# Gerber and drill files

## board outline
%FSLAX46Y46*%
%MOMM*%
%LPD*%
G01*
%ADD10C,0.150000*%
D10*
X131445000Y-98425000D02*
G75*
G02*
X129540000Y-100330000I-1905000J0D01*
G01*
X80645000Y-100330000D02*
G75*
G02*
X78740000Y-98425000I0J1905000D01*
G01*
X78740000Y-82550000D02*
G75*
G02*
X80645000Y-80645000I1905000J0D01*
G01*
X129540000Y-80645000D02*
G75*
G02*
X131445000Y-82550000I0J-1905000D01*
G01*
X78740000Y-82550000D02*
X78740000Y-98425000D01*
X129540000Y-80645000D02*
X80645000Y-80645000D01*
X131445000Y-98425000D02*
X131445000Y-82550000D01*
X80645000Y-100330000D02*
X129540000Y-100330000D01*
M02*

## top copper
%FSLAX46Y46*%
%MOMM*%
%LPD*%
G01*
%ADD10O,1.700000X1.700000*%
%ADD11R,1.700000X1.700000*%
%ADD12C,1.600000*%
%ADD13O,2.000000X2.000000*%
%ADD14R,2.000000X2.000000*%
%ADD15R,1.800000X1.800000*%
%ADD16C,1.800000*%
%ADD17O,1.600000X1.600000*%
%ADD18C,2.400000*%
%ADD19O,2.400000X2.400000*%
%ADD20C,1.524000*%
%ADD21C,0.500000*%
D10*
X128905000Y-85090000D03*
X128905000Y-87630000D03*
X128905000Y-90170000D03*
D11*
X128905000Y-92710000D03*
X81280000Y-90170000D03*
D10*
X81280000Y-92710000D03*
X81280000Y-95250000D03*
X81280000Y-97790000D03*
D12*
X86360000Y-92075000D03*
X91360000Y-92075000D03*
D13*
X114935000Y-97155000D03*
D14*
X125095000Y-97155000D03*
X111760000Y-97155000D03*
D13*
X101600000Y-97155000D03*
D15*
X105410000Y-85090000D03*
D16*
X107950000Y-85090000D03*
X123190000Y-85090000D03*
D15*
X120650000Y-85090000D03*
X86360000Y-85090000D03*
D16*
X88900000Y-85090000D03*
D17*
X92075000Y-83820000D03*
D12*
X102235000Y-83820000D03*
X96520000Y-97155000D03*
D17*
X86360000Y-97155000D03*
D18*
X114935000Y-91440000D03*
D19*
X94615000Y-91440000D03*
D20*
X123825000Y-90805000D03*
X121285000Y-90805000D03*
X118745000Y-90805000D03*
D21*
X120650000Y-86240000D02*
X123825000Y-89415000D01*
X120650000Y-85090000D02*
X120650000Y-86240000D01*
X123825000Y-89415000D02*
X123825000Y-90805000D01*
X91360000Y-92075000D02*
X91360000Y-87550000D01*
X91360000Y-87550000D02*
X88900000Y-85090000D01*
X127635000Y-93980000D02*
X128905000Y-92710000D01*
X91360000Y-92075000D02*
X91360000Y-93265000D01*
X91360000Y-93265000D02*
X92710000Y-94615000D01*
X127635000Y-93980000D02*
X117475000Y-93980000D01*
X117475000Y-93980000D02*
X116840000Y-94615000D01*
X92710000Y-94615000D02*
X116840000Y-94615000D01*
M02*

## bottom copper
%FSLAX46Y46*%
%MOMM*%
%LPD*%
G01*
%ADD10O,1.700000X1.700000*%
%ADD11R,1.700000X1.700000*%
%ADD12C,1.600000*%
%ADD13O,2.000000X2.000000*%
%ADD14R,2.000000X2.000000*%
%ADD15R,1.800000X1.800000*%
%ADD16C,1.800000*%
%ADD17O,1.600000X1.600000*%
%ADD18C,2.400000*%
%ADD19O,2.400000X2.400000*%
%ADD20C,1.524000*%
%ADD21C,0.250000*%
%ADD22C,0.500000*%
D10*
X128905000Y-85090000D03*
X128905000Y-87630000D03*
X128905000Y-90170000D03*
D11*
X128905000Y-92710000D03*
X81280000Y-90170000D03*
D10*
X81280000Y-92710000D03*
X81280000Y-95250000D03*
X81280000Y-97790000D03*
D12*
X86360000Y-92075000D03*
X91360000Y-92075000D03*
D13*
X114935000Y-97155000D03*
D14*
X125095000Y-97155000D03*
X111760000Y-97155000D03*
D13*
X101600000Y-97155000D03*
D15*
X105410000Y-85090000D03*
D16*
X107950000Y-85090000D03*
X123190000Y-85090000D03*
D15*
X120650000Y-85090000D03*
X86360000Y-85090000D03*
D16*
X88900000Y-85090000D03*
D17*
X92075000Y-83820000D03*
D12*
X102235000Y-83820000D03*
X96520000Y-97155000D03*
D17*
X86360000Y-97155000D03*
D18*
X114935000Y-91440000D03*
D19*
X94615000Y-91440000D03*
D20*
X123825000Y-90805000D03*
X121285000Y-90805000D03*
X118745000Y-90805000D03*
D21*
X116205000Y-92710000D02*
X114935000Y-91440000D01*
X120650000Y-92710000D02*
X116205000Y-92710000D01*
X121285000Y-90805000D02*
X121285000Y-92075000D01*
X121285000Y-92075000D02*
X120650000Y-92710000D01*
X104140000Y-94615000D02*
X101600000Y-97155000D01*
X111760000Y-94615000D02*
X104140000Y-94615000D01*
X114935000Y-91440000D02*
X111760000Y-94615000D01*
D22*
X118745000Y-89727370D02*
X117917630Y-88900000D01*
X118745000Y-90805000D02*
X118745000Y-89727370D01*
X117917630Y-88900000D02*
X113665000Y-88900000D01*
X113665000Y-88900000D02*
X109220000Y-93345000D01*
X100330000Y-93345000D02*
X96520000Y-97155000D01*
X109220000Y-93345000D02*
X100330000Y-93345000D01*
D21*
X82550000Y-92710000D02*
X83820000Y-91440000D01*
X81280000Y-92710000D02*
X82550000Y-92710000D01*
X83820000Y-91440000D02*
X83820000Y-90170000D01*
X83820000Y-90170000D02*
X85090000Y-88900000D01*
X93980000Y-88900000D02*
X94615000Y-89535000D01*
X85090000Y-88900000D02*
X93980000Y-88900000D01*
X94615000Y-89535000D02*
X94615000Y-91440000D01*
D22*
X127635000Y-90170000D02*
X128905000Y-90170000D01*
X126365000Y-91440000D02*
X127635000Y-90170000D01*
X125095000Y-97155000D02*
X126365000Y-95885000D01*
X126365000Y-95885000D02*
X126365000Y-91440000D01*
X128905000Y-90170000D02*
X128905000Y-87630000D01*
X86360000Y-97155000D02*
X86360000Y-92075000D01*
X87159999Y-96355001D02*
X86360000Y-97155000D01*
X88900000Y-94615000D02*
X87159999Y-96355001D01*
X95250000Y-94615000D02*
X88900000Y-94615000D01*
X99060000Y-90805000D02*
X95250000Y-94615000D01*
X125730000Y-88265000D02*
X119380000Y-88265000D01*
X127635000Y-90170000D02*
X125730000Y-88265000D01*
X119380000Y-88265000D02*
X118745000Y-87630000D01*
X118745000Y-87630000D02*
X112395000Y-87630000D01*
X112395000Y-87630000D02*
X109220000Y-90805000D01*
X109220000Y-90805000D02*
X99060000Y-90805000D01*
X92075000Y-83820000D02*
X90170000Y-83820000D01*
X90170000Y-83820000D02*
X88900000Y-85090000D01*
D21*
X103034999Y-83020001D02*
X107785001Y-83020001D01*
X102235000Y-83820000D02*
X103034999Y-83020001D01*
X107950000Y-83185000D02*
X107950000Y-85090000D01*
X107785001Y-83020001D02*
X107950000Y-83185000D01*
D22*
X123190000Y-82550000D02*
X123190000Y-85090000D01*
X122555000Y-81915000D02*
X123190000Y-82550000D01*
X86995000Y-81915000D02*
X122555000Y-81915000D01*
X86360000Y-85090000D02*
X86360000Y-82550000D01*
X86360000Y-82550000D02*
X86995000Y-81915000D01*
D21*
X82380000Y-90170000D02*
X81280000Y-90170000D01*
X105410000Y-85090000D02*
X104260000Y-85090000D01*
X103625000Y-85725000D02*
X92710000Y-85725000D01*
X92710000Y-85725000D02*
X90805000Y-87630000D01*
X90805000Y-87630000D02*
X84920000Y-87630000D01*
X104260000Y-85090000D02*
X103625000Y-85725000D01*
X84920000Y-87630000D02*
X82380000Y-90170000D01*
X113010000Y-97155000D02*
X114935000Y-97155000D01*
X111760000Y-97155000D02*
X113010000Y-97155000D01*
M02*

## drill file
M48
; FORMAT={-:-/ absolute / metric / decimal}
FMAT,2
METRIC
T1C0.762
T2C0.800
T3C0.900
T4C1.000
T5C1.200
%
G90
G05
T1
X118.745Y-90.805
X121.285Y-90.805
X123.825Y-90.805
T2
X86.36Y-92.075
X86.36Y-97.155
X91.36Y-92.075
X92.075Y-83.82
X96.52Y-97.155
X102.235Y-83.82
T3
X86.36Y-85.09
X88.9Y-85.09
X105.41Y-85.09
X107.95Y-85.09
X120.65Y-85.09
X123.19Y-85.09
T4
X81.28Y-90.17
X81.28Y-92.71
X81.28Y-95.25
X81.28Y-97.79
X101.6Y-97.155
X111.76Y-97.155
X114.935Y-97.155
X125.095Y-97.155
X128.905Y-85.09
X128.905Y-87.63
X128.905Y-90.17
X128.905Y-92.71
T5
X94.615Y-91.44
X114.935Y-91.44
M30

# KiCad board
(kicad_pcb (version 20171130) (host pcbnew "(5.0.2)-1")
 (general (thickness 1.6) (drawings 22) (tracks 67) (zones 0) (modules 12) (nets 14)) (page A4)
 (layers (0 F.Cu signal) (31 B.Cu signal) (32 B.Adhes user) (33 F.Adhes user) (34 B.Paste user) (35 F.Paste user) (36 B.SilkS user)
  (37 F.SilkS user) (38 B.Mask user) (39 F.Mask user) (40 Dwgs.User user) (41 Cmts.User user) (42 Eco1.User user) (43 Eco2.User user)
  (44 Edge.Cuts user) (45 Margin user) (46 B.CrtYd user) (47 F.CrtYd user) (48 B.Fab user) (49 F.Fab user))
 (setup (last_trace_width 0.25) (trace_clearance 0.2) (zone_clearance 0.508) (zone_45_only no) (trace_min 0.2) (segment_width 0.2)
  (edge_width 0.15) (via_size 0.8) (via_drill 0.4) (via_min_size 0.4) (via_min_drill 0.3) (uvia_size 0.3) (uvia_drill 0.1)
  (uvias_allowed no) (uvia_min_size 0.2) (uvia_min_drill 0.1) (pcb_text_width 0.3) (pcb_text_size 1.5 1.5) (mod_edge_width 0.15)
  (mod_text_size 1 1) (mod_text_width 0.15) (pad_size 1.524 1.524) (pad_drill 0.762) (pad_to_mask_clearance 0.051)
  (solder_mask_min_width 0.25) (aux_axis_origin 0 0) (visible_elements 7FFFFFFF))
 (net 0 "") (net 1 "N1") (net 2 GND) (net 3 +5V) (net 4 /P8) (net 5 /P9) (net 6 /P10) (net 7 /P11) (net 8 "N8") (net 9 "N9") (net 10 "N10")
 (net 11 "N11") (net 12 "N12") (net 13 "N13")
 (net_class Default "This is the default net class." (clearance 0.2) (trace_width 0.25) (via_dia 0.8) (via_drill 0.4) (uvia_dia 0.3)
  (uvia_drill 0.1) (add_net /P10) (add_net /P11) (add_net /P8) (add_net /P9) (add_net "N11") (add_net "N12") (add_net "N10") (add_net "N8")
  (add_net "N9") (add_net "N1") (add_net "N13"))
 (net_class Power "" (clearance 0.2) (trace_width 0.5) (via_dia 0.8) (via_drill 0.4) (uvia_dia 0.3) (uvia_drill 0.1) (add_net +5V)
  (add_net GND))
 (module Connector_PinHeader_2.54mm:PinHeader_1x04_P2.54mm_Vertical (layer B.Cu) (at 128.905 92.71)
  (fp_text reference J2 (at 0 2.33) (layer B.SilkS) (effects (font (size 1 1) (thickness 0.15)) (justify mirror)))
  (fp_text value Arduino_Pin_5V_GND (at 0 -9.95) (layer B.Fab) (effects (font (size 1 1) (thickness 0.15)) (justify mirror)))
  (pad 4 thru_hole oval (at 0 -7.62) (size 1.7 1.7) (drill 1) (layers *.Cu *.Mask) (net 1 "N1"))
  (pad 3 thru_hole oval (at 0 -5.08) (size 1.7 1.7) (drill 1) (layers *.Cu *.Mask) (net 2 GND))
  (pad 2 thru_hole oval (at 0 -2.54) (size 1.7 1.7) (drill 1) (layers *.Cu *.Mask) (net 2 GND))
  (pad 1 thru_hole rect (at 0 0) (size 1.7 1.7) (drill 1) (layers *.Cu *.Mask) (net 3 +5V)))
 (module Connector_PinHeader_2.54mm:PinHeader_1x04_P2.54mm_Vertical (layer B.Cu) (at 81.28 90.17 180)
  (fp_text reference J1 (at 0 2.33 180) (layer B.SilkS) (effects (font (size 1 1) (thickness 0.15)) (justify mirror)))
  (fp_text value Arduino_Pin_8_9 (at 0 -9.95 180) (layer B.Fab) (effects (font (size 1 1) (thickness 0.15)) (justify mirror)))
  (pad 1 thru_hole rect (at 0 0 180) (size 1.7 1.7) (drill 1) (layers *.Cu *.Mask) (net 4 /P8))
  (pad 2 thru_hole oval (at 0 -2.54 180) (size 1.7 1.7) (drill 1) (layers *.Cu *.Mask) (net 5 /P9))
  (pad 3 thru_hole oval (at 0 -5.08 180) (size 1.7 1.7) (drill 1) (layers *.Cu *.Mask) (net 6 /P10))
  (pad 4 thru_hole oval (at 0 -7.62 180) (size 1.7 1.7) (drill 1) (layers *.Cu *.Mask) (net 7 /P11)))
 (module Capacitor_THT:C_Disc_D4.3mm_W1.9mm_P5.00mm (layer F.Cu) (at 86.36 92.075)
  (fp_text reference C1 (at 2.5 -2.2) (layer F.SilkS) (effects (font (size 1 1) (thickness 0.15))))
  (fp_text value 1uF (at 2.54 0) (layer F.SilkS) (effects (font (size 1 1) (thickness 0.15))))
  (pad 1 thru_hole circle (at 0 0) (size 1.6 1.6) (drill 0.8) (layers *.Cu *.Mask) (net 2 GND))
  (pad 2 thru_hole circle (at 5 0) (size 1.6 1.6) (drill 0.8) (layers *.Cu *.Mask) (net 3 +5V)))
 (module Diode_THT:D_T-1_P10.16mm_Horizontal (layer F.Cu) (at 125.095 97.155 180)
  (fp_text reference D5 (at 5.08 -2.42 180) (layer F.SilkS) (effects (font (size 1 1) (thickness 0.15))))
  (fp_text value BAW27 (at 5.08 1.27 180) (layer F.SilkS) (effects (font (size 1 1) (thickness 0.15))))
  (pad 2 thru_hole oval (at 10.16 0 180) (size 2 2) (drill 1) (layers *.Cu *.Mask) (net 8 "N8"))
  (pad 1 thru_hole rect (at 0 0 180) (size 2 2) (drill 1) (layers *.Cu *.Mask) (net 2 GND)))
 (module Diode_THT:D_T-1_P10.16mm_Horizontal (layer F.Cu) (at 111.76 97.155 180)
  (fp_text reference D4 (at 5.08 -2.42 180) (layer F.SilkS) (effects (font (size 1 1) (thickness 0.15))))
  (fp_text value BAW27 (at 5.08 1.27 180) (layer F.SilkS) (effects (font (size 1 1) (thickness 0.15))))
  (pad 1 thru_hole rect (at 0 0 180) (size 2 2) (drill 1) (layers *.Cu *.Mask) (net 8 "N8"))
  (pad 2 thru_hole oval (at 10.16 0 180) (size 2 2) (drill 1) (layers *.Cu *.Mask) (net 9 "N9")))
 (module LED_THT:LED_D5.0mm (layer F.Cu) (at 105.41 85.09)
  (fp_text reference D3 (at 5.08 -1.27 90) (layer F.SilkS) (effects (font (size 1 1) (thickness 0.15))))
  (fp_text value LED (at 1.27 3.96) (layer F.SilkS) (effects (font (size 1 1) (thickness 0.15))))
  (pad 1 thru_hole rect (at 0 0) (size 1.8 1.8) (drill 0.9) (layers *.Cu *.Mask) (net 4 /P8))
  (pad 2 thru_hole circle (at 2.54 0) (size 1.8 1.8) (drill 0.9) (layers *.Cu *.Mask) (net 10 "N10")))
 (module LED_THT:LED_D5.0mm (layer B.Cu) (at 120.65 85.09)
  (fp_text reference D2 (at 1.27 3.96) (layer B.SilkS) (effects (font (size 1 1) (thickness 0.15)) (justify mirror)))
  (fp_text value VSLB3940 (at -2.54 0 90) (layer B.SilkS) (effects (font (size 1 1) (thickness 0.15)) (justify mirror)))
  (pad 2 thru_hole circle (at 2.54 0) (size 1.8 1.8) (drill 0.9) (layers *.Cu *.Mask) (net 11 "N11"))
  (pad 1 thru_hole rect (at 0 0) (size 1.8 1.8) (drill 0.9) (layers *.Cu *.Mask) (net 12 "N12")))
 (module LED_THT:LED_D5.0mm (layer B.Cu) (at 86.36 85.09)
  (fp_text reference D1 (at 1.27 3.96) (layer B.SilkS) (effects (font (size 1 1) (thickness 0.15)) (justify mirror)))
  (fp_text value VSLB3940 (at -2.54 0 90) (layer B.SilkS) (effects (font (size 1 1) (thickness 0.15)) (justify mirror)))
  (pad 1 thru_hole rect (at 0 0) (size 1.8 1.8) (drill 0.9) (layers *.Cu *.Mask) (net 11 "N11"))
  (pad 2 thru_hole circle (at 2.54 0) (size 1.8 1.8) (drill 0.9) (layers *.Cu *.Mask) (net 3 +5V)))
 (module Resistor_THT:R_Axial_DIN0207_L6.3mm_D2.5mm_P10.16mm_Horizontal (layer F.Cu) (at 102.235 83.82 180)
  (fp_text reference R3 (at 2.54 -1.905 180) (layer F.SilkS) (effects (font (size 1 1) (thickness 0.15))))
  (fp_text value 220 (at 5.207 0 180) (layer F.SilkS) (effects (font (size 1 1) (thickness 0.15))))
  (pad 2 thru_hole oval (at 10.16 0 180) (size 1.6 1.6) (drill 0.8) (layers *.Cu *.Mask) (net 3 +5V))
  (pad 1 thru_hole circle (at 0 0 180) (size 1.6 1.6) (drill 0.8) (layers *.Cu *.Mask) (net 10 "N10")))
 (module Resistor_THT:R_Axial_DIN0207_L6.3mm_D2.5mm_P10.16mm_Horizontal (layer F.Cu) (at 96.52 97.155 180)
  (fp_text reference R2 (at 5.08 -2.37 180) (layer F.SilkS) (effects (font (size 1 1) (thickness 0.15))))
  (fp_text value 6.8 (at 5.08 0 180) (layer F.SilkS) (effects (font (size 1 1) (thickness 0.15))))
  (pad 1 thru_hole circle (at 0 0 180) (size 1.6 1.6) (drill 0.8) (layers *.Cu *.Mask) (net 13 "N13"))
  (pad 2 thru_hole oval (at 10.16 0 180) (size 1.6 1.6) (drill 0.8) (layers *.Cu *.Mask) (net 2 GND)))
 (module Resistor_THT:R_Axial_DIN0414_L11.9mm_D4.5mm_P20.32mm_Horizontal (layer F.Cu) (at 114.935 91.44 180)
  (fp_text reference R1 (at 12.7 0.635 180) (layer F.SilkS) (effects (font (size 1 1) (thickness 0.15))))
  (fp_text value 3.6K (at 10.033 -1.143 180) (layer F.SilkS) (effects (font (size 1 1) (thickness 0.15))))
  (pad 1 thru_hole circle (at 0 0 180) (size 2.4 2.4) (drill 1.2) (layers *.Cu *.Mask) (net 9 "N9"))
  (pad 2 thru_hole oval (at 20.32 0 180) (size 2.4 2.4) (drill 1.2) (layers *.Cu *.Mask) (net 5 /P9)))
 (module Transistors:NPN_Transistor (layer F.Cu) (at 123.825 90.805 180)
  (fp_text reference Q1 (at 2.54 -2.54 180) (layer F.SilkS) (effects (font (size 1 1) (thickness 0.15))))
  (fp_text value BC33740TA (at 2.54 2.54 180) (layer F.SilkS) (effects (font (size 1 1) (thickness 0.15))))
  (pad 1 thru_hole circle (at 0 0 180) (size 1.524 1.524) (drill 0.762) (layers *.Cu *.Mask) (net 12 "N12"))
  (pad 2 thru_hole circle (at 2.54 0 180) (size 1.524 1.524) (drill 0.762) (layers *.Cu *.Mask) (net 9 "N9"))
  (pad 3 thru_hole circle (at 5.08 0 180) (size 1.524 1.524) (drill 0.762) (layers *.Cu *.Mask) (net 13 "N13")))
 (gr_arc (start 129.54 98.425) (end 129.54 100.33) (angle -90) (layer Edge.Cuts) (width 0.15))
 (gr_arc (start 80.645 98.425) (end 78.74 98.425) (angle -90) (layer Edge.Cuts) (width 0.15))
 (gr_arc (start 80.645 82.55) (end 80.645 80.645) (angle -90) (layer Edge.Cuts) (width 0.15))
 (gr_arc (start 129.54 82.55) (end 131.445 82.55) (angle -90) (layer Edge.Cuts) (width 0.15))
 (gr_line (start 78.74 82.55) (end 78.74 98.425) (layer Edge.Cuts) (width 0.15))
 (gr_line (start 129.54 80.645) (end 80.645 80.645) (layer Edge.Cuts) (width 0.15))
 (gr_line (start 131.445 98.425) (end 131.445 82.55) (layer Edge.Cuts) (width 0.15))
 (gr_line (start 80.645 100.33) (end 129.54 100.33) (layer Edge.Cuts) (width 0.15))
 (segment (start 120.65 86.24) (end 123.825 89.415) (width 0.5) (layer F.Cu) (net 12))
 (segment (start 120.65 85.09) (end 120.65 86.24) (width 0.5) (layer F.Cu) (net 12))
 (segment (start 123.825 89.415) (end 123.825 90.805) (width 0.5) (layer F.Cu) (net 12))
 (segment (start 116.205 92.71) (end 114.935 91.44) (width 0.25) (layer B.Cu) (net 9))
 (segment (start 120.65 92.71) (end 116.205 92.71) (width 0.25) (layer B.Cu) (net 9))
 (segment (start 121.285 90.805) (end 121.285 92.075) (width 0.25) (layer B.Cu) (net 9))
 (segment (start 121.285 92.075) (end 120.65 92.71) (width 0.25) (layer B.Cu) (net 9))
 (segment (start 104.14 94.615) (end 101.6 97.155) (width 0.25) (layer B.Cu) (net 9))
 (segment (start 111.76 94.615) (end 104.14 94.615) (width 0.25) (layer B.Cu) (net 9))
 (segment (start 114.935 91.44) (end 111.76 94.615) (width 0.25) (layer B.Cu) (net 9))
 (segment (start 118.745 89.72737) (end 117.91763 88.9) (width 0.5) (layer B.Cu) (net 13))
 (segment (start 118.745 90.805) (end 118.745 89.72737) (width 0.5) (layer B.Cu) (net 13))
 (segment (start 117.91763 88.9) (end 113.665 88.9) (width 0.5) (layer B.Cu) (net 13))
 (segment (start 113.665 88.9) (end 109.22 93.345) (width 0.5) (layer B.Cu) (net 13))
 (segment (start 100.33 93.345) (end 96.52 97.155) (width 0.5) (layer B.Cu) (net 13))
 (segment (start 109.22 93.345) (end 100.33 93.345) (width 0.5) (layer B.Cu) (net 13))
 (segment (start 82.55 92.71) (end 83.82 91.44) (width 0.25) (layer B.Cu) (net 5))
 (segment (start 81.28 92.71) (end 82.55 92.71) (width 0.25) (layer B.Cu) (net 5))
 (segment (start 83.82 91.44) (end 83.82 90.17) (width 0.25) (layer B.Cu) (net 5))
 (segment (start 83.82 90.17) (end 85.09 88.9) (width 0.25) (layer B.Cu) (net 5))
 (segment (start 93.98 88.9) (end 94.615 89.535) (width 0.25) (layer B.Cu) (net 5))
 (segment (start 85.09 88.9) (end 93.98 88.9) (width 0.25) (layer B.Cu) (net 5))
 (segment (start 94.615 89.535) (end 94.615 91.44) (width 0.25) (layer B.Cu) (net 5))
 (segment (start 127.635 90.17) (end 128.905 90.17) (width 0.5) (layer B.Cu) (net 2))
 (segment (start 126.365 91.44) (end 127.635 90.17) (width 0.5) (layer B.Cu) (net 2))
 (segment (start 125.095 97.155) (end 126.365 95.885) (width 0.5) (layer B.Cu) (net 2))
 (segment (start 126.365 95.885) (end 126.365 91.44) (width 0.5) (layer B.Cu) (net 2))
 (segment (start 128.905 90.17) (end 128.905 87.63) (width 0.5) (layer B.Cu) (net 2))
 (segment (start 86.36 97.155) (end 86.36 92.075) (width 0.5) (layer B.Cu) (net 2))
 (segment (start 87.159999 96.355001) (end 86.36 97.155) (width 0.5) (layer B.Cu) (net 2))
 (segment (start 88.9 94.615) (end 87.159999 96.355001) (width 0.5) (layer B.Cu) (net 2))
 (segment (start 95.25 94.615) (end 88.9 94.615) (width 0.5) (layer B.Cu) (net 2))
 (segment (start 99.06 90.805) (end 95.25 94.615) (width 0.5) (layer B.Cu) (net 2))
 (segment (start 125.73 88.265) (end 119.38 88.265) (width 0.5) (layer B.Cu) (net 2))
 (segment (start 127.635 90.17) (end 125.73 88.265) (width 0.5) (layer B.Cu) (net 2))
 (segment (start 119.38 88.265) (end 118.745 87.63) (width 0.5) (layer B.Cu) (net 2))
 (segment (start 118.745 87.63) (end 112.395 87.63) (width 0.5) (layer B.Cu) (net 2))
 (segment (start 112.395 87.63) (end 109.22 90.805) (width 0.5) (layer B.Cu) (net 2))
 (segment (start 109.22 90.805) (end 99.06 90.805) (width 0.5) (layer B.Cu) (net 2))
 (segment (start 91.36 92.075) (end 91.36 87.55) (width 0.5) (layer F.Cu) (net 3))
 (segment (start 91.36 87.55) (end 88.9 85.09) (width 0.5) (layer F.Cu) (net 3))
 (segment (start 92.075 83.82) (end 90.17 83.82) (width 0.5) (layer B.Cu) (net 3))
 (segment (start 90.17 83.82) (end 88.9 85.09) (width 0.5) (layer B.Cu) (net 3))
 (segment (start 127.635 93.98) (end 128.905 92.71) (width 0.5) (layer F.Cu) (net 3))
 (segment (start 91.36 92.075) (end 91.36 93.265) (width 0.5) (layer F.Cu) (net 3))
 (segment (start 91.36 93.265) (end 92.71 94.615) (width 0.5) (layer F.Cu) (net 3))
 (segment (start 127.635 93.98) (end 117.475 93.98) (width 0.5) (layer F.Cu) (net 3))
 (segment (start 117.475 93.98) (end 116.84 94.615) (width 0.5) (layer F.Cu) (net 3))
 (segment (start 92.71 94.615) (end 116.84 94.615) (width 0.5) (layer F.Cu) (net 3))
 (segment (start 103.034999 83.020001) (end 107.785001 83.020001) (width 0.25) (layer B.Cu) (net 10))
 (segment (start 102.235 83.82) (end 103.034999 83.020001) (width 0.25) (layer B.Cu) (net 10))
 (segment (start 107.95 83.185) (end 107.95 85.09) (width 0.25) (layer B.Cu) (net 10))
 (segment (start 107.785001 83.020001) (end 107.95 83.185) (width 0.25) (layer B.Cu) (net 10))
 (segment (start 123.19 82.55) (end 123.19 85.09) (width 0.5) (layer B.Cu) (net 11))
 (segment (start 122.555 81.915) (end 123.19 82.55) (width 0.5) (layer B.Cu) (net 11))
 (segment (start 86.995 81.915) (end 122.555 81.915) (width 0.5) (layer B.Cu) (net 11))
 (segment (start 86.36 85.09) (end 86.36 82.55) (width 0.5) (layer B.Cu) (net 11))
 (segment (start 86.36 82.55) (end 86.995 81.915) (width 0.5) (layer B.Cu) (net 11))
 (segment (start 82.38 90.17) (end 81.28 90.17) (width 0.25) (layer B.Cu) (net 4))
 (segment (start 105.41 85.09) (end 104.26 85.09) (width 0.25) (layer B.Cu) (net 4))
 (segment (start 103.625 85.725) (end 92.71 85.725) (width 0.25) (layer B.Cu) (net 4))
 (segment (start 92.71 85.725) (end 90.805 87.63) (width 0.25) (layer B.Cu) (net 4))
 (segment (start 90.805 87.63) (end 84.92 87.63) (width 0.25) (layer B.Cu) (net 4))
 (segment (start 104.26 85.09) (end 103.625 85.725) (width 0.25) (layer B.Cu) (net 4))
 (segment (start 84.92 87.63) (end 82.38 90.17) (width 0.25) (layer B.Cu) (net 4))
 (segment (start 113.01 97.155) (end 114.935 97.155) (width 0.25) (layer B.Cu) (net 8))
 (segment (start 111.76 97.155) (end 113.01 97.155) (width 0.25) (layer B.Cu) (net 8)))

